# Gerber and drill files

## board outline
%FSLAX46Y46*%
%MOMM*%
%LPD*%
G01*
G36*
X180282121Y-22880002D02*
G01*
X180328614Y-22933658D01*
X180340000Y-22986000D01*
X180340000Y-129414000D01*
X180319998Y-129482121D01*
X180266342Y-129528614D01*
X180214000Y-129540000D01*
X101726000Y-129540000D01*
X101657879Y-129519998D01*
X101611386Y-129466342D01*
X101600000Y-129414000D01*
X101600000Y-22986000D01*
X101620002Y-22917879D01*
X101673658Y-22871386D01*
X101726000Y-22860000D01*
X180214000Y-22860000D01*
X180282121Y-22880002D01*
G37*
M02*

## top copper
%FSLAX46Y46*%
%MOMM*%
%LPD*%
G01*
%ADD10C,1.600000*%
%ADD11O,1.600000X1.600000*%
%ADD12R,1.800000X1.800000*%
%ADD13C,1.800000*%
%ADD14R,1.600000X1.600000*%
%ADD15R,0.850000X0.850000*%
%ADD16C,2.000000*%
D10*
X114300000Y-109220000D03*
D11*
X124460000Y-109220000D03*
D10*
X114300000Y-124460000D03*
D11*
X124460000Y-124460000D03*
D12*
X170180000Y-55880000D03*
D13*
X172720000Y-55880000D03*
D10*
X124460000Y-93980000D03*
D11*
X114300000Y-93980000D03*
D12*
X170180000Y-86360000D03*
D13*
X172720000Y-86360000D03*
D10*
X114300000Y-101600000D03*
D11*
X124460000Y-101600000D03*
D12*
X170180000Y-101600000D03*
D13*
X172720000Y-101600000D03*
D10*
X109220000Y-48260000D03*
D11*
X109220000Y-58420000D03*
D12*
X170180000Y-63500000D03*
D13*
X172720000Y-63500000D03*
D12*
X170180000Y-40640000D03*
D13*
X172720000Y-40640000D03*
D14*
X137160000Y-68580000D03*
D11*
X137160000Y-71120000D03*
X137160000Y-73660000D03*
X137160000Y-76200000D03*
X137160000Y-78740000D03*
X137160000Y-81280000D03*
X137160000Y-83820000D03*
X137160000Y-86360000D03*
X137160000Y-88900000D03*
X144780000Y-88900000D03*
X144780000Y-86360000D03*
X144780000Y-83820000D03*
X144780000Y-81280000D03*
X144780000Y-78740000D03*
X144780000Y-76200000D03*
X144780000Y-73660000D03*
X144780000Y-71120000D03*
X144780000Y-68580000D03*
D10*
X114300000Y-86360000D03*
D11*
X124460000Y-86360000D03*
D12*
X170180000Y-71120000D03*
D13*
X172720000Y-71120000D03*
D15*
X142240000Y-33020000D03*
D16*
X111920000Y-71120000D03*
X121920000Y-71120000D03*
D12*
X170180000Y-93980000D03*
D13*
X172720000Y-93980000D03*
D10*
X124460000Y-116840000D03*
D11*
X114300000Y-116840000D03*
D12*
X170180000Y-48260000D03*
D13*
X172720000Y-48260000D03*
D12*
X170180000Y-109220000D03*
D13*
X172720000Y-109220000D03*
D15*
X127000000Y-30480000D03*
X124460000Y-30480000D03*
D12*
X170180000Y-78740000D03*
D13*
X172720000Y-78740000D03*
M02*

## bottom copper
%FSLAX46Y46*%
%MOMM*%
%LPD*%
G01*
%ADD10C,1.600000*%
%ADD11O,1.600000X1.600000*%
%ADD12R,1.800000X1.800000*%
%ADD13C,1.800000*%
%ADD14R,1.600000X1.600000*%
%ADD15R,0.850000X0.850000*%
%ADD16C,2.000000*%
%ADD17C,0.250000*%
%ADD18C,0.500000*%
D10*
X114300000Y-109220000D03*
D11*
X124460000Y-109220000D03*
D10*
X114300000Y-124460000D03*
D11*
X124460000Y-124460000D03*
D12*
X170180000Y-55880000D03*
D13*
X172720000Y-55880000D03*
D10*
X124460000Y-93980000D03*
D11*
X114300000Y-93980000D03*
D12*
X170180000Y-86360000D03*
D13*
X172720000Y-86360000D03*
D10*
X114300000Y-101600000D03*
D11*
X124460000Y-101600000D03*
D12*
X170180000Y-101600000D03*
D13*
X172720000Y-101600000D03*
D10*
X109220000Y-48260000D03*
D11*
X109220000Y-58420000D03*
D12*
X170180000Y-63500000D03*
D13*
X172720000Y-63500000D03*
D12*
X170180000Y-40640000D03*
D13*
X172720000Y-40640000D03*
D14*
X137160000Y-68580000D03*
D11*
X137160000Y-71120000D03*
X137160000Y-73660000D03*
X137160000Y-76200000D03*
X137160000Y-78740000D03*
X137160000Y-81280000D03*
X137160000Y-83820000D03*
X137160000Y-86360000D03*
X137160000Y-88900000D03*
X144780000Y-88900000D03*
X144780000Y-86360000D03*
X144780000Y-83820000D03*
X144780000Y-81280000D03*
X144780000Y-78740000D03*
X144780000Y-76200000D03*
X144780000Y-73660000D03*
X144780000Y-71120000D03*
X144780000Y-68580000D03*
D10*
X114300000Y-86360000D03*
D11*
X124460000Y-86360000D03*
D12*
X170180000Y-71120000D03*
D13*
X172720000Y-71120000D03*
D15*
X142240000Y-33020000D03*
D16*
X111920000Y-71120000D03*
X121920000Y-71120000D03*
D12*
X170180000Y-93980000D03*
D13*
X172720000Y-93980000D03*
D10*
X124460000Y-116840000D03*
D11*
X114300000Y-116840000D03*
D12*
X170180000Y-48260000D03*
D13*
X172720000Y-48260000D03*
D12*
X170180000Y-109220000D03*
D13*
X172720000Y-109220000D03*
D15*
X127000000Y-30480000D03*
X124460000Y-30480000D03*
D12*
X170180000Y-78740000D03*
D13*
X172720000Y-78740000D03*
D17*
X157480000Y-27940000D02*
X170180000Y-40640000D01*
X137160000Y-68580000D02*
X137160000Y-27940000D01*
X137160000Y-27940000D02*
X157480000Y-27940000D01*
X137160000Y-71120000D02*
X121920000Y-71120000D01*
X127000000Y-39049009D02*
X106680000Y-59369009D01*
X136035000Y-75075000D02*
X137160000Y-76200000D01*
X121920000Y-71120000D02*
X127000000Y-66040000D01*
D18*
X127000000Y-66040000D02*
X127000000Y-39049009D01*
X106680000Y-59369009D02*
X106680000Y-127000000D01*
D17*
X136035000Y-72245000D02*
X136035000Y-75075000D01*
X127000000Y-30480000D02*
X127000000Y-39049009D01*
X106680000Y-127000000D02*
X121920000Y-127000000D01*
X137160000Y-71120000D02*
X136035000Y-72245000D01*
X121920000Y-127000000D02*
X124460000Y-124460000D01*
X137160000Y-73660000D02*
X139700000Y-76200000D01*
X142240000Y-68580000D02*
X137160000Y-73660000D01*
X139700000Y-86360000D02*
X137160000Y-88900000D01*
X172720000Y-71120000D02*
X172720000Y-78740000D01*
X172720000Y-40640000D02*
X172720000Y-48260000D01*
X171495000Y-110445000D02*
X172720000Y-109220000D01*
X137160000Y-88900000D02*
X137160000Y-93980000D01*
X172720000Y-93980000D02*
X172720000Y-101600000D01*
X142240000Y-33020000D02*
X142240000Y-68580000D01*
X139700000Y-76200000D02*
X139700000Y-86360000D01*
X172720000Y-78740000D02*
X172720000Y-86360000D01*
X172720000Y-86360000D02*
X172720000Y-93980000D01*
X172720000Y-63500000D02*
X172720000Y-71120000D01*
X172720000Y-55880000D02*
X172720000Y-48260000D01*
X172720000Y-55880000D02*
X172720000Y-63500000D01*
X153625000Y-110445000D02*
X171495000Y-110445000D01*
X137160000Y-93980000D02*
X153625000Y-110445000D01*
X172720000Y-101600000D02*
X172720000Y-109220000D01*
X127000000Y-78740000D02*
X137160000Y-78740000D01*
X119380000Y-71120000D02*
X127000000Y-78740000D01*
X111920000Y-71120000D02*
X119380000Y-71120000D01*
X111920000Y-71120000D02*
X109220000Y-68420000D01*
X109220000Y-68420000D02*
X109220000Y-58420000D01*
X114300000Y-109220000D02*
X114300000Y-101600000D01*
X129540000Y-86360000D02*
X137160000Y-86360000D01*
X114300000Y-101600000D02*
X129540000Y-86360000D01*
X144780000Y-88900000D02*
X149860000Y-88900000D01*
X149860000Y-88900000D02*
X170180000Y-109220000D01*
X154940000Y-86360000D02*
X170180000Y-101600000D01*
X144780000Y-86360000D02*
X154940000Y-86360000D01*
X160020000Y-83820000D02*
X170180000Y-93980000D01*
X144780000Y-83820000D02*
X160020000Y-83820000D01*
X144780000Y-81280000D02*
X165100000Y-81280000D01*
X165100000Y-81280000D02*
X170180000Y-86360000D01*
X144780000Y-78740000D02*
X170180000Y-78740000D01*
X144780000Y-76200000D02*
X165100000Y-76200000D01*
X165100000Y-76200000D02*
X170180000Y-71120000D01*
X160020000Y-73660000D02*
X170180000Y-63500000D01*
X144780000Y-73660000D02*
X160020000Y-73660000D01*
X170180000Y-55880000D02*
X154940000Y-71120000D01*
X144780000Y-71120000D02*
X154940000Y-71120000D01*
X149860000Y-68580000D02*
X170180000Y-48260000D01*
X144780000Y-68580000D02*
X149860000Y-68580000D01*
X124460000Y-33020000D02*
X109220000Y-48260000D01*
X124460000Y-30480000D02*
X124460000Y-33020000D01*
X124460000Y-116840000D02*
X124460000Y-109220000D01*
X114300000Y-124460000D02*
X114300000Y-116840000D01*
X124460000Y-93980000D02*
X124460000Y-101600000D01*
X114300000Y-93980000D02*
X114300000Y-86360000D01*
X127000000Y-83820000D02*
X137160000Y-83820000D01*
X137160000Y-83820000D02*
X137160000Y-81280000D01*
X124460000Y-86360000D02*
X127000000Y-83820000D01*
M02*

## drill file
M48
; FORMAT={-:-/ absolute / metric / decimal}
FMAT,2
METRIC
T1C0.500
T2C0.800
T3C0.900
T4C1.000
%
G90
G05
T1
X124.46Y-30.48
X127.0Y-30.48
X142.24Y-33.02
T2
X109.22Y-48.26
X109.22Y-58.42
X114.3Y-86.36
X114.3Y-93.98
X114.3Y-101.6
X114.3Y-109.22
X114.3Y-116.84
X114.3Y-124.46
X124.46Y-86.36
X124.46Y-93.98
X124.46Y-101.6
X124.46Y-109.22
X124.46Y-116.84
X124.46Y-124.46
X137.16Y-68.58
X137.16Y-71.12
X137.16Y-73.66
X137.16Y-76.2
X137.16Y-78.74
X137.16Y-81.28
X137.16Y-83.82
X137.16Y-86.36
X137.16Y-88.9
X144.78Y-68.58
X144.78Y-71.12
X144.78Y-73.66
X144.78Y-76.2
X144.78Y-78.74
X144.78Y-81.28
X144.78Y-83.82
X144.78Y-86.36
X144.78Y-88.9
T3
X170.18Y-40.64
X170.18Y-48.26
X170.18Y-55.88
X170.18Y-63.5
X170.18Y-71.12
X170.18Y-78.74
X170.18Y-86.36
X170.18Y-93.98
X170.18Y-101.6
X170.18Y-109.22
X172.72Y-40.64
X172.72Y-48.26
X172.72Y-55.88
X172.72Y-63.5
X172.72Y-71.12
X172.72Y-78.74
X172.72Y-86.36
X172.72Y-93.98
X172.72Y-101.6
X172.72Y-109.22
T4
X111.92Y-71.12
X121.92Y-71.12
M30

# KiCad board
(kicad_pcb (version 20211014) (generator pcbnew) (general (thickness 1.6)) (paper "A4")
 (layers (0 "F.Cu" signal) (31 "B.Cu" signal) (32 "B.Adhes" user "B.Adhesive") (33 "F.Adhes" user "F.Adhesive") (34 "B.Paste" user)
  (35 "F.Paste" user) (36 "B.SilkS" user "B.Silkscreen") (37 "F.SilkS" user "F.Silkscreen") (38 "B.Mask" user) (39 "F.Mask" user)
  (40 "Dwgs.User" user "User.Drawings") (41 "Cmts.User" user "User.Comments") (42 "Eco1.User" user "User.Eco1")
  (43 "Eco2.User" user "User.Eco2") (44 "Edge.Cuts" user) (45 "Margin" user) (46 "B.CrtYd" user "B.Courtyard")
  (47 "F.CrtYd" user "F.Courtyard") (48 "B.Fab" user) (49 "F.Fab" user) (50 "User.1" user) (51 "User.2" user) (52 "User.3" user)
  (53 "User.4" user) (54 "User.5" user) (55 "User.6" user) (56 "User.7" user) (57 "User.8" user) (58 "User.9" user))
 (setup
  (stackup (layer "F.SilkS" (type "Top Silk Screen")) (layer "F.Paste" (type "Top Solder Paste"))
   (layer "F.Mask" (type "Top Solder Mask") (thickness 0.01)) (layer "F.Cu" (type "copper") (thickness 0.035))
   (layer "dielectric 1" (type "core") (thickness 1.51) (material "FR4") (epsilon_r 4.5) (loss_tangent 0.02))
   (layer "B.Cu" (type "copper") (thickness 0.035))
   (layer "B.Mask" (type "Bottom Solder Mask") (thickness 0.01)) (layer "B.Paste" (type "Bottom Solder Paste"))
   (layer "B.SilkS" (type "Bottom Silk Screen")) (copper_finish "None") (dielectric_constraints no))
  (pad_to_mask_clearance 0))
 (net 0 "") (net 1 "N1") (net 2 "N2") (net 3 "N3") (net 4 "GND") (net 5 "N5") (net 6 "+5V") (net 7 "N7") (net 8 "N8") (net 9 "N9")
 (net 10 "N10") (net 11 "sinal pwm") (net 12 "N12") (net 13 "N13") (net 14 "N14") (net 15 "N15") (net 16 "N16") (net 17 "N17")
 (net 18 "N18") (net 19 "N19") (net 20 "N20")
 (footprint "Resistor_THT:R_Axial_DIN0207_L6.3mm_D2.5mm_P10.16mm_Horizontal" (layer "F.Cu") (at 114.3 109.22)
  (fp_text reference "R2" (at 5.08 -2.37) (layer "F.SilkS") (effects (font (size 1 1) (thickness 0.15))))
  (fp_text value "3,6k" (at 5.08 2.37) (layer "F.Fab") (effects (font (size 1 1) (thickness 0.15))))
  (pad "1" thru_hole circle (at 0 0) (size 1.6 1.6) (drill 0.8) (layers *.Cu *.Mask) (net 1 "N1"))
  (pad "2" thru_hole oval (at 10.16 0) (size 1.6 1.6) (drill 0.8) (layers *.Cu *.Mask) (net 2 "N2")))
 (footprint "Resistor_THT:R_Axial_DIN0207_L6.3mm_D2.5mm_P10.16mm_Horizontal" (layer "F.Cu") (at 114.3 124.46)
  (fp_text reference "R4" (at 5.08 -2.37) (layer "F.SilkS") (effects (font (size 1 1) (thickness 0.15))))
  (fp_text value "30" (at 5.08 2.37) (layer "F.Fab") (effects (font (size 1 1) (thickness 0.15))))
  (pad "1" thru_hole circle (at 0 0) (size 1.6 1.6) (drill 0.8) (layers *.Cu *.Mask) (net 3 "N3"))
  (pad "2" thru_hole oval (at 10.16 0) (size 1.6 1.6) (drill 0.8) (layers *.Cu *.Mask) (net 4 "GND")))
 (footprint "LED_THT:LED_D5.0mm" (layer "F.Cu") (at 170.18 55.88)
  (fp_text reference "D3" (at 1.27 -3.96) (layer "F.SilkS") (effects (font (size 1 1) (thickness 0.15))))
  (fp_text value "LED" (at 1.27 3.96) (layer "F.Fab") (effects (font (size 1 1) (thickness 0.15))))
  (pad "1" thru_hole rect (at 0 0) (size 1.8 1.8) (drill 0.9) (layers *.Cu *.Mask) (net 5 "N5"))
  (pad "2" thru_hole circle (at 2.54 0) (size 1.8 1.8) (drill 0.9) (layers *.Cu *.Mask) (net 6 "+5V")))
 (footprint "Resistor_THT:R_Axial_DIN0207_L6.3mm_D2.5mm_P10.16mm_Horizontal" (layer "F.Cu") (at 124.46 93.98 180)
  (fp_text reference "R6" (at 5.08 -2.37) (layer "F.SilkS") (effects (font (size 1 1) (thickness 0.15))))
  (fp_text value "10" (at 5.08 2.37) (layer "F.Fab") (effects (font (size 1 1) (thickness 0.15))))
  (pad "1" thru_hole circle (at 0 0 180) (size 1.6 1.6) (drill 0.8) (layers *.Cu *.Mask) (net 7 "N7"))
  (pad "2" thru_hole oval (at 10.16 0 180) (size 1.6 1.6) (drill 0.8) (layers *.Cu *.Mask) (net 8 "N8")))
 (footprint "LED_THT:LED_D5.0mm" (layer "F.Cu") (at 170.18 86.36)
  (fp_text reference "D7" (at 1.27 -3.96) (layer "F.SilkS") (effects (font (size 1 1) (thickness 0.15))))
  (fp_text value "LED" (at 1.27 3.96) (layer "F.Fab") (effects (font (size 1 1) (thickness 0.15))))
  (pad "1" thru_hole rect (at 0 0) (size 1.8 1.8) (drill 0.9) (layers *.Cu *.Mask) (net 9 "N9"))
  (pad "2" thru_hole circle (at 2.54 0) (size 1.8 1.8) (drill 0.9) (layers *.Cu *.Mask) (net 6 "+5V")))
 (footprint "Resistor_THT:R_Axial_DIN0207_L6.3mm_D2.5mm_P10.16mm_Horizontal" (layer "F.Cu") (at 114.3 101.6)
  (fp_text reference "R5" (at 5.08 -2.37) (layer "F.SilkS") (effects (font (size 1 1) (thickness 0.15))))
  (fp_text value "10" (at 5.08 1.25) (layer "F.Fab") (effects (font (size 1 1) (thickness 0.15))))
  (pad "1" thru_hole circle (at 0 0) (size 1.6 1.6) (drill 0.8) (layers *.Cu *.Mask) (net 1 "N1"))
  (pad "2" thru_hole oval (at 10.16 0) (size 1.6 1.6) (drill 0.8) (layers *.Cu *.Mask) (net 7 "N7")))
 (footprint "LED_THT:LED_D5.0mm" (layer "F.Cu") (at 170.18 101.6)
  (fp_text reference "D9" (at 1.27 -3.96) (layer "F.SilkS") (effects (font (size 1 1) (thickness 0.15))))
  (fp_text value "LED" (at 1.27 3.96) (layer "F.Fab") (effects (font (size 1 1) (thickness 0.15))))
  (pad "1" thru_hole rect (at 0 0) (size 1.8 1.8) (drill 0.9) (layers *.Cu *.Mask) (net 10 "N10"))
  (pad "2" thru_hole circle (at 2.54 0) (size 1.8 1.8) (drill 0.9) (layers *.Cu *.Mask) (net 6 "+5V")))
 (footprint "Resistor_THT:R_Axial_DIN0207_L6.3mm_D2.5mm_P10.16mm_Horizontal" (layer "F.Cu") (at 109.22 48.26 -90)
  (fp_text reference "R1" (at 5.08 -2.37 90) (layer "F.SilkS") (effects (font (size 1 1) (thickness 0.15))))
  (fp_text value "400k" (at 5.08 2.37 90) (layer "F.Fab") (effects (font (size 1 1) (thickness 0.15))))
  (pad "1" thru_hole circle (at 0 0 270) (size 1.6 1.6) (drill 0.8) (layers *.Cu *.Mask) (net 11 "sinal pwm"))
  (pad "2" thru_hole oval (at 10.16 0 270) (size 1.6 1.6) (drill 0.8) (layers *.Cu *.Mask) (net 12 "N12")))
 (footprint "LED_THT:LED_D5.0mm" (layer "F.Cu") (at 170.18 63.5)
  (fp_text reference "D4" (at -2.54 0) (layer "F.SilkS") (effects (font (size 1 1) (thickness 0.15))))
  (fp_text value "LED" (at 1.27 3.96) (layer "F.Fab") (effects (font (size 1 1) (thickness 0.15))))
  (pad "1" thru_hole rect (at 0 0) (size 1.8 1.8) (drill 0.9) (layers *.Cu *.Mask) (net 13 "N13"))
  (pad "2" thru_hole circle (at 2.54 0) (size 1.8 1.8) (drill 0.9) (layers *.Cu *.Mask) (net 6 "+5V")))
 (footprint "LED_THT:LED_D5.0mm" (layer "F.Cu") (at 170.18 40.64)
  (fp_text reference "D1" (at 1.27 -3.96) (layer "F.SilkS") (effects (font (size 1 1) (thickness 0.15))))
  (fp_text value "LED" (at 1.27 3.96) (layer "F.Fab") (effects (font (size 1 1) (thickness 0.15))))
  (pad "1" thru_hole rect (at 0 0) (size 1.8 1.8) (drill 0.9) (layers *.Cu *.Mask) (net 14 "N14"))
  (pad "2" thru_hole circle (at 2.54 0) (size 1.8 1.8) (drill 0.9) (layers *.Cu *.Mask) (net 6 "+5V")))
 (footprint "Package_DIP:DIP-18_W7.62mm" (layer "F.Cu") (at 137.16 68.58)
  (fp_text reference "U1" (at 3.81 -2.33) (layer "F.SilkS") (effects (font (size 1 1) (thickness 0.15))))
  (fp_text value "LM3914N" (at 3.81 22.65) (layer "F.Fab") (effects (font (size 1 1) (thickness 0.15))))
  (pad "1" thru_hole rect (at 0 0) (size 1.6 1.6) (drill 0.8) (layers *.Cu *.Mask) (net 14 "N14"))
  (pad "2" thru_hole oval (at 0 2.54) (size 1.6 1.6) (drill 0.8) (layers *.Cu *.Mask) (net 4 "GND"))
  (pad "3" thru_hole oval (at 0 5.08) (size 1.6 1.6) (drill 0.8) (layers *.Cu *.Mask) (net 6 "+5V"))
  (pad "4" thru_hole oval (at 0 7.62) (size 1.6 1.6) (drill 0.8) (layers *.Cu *.Mask) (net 4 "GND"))
  (pad "5" thru_hole oval (at 0 10.16) (size 1.6 1.6) (drill 0.8) (layers *.Cu *.Mask) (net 12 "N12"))
  (pad "6" thru_hole oval (at 0 12.7) (size 1.6 1.6) (drill 0.8) (layers *.Cu *.Mask) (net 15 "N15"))
  (pad "7" thru_hole oval (at 0 15.24) (size 1.6 1.6) (drill 0.8) (layers *.Cu *.Mask) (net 15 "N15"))
  (pad "8" thru_hole oval (at 0 17.78) (size 1.6 1.6) (drill 0.8) (layers *.Cu *.Mask) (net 1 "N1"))
  (pad "9" thru_hole oval (at 0 20.32) (size 1.6 1.6) (drill 0.8) (layers *.Cu *.Mask) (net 6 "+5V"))
  (pad "10" thru_hole oval (at 7.62 20.32) (size 1.6 1.6) (drill 0.8) (layers *.Cu *.Mask) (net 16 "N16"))
  (pad "11" thru_hole oval (at 7.62 17.78) (size 1.6 1.6) (drill 0.8) (layers *.Cu *.Mask) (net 10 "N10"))
  (pad "12" thru_hole oval (at 7.62 15.24) (size 1.6 1.6) (drill 0.8) (layers *.Cu *.Mask) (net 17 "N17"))
  (pad "13" thru_hole oval (at 7.62 12.7) (size 1.6 1.6) (drill 0.8) (layers *.Cu *.Mask) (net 9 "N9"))
  (pad "14" thru_hole oval (at 7.62 10.16) (size 1.6 1.6) (drill 0.8) (layers *.Cu *.Mask) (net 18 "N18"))
  (pad "15" thru_hole oval (at 7.62 7.62) (size 1.6 1.6) (drill 0.8) (layers *.Cu *.Mask) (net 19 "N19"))
  (pad "16" thru_hole oval (at 7.62 5.08) (size 1.6 1.6) (drill 0.8) (layers *.Cu *.Mask) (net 13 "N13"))
  (pad "17" thru_hole oval (at 7.62 2.54) (size 1.6 1.6) (drill 0.8) (layers *.Cu *.Mask) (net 5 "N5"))
  (pad "18" thru_hole oval (at 7.62 0) (size 1.6 1.6) (drill 0.8) (layers *.Cu *.Mask) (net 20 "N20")))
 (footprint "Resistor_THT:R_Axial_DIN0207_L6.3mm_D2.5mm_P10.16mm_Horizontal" (layer "F.Cu") (at 114.3 86.36)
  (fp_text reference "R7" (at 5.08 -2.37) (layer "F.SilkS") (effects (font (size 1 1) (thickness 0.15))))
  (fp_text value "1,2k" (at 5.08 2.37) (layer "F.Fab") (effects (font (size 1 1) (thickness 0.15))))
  (pad "1" thru_hole circle (at 0 0) (size 1.6 1.6) (drill 0.8) (layers *.Cu *.Mask) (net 8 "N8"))
  (pad "2" thru_hole oval (at 10.16 0) (size 1.6 1.6) (drill 0.8) (layers *.Cu *.Mask) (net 15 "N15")))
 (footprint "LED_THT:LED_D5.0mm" (layer "F.Cu") (at 170.18 71.12)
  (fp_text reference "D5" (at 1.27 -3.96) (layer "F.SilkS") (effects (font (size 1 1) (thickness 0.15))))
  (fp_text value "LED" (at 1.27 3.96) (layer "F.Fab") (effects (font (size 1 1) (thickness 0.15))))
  (pad "1" thru_hole rect (at 0 0) (size 1.8 1.8) (drill 0.9) (layers *.Cu *.Mask) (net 19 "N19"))
  (pad "2" thru_hole circle (at 2.54 0) (size 1.8 1.8) (drill 0.9) (layers *.Cu *.Mask) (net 6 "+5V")))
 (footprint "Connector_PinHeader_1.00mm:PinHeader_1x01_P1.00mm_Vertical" (layer "F.Cu") (at 142.24 33.02)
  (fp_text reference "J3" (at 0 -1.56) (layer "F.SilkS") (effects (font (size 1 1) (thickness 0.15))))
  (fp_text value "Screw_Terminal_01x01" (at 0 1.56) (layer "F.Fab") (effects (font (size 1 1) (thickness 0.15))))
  (pad "1" thru_hole rect (at 0 0) (size 0.85 0.85) (drill 0.5) (layers *.Cu *.Mask) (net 6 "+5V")))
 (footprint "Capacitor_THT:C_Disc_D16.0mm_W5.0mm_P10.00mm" (layer "F.Cu") (at 111.92 71.12)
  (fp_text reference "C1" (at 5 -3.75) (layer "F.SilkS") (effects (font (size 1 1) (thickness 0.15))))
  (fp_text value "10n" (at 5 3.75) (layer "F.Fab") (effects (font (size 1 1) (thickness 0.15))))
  (pad "1" thru_hole circle (at 0 0) (size 2 2) (drill 1) (layers *.Cu *.Mask) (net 12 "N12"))
  (pad "2" thru_hole circle (at 10 0) (size 2 2) (drill 1) (layers *.Cu *.Mask) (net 4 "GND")))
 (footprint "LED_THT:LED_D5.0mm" (layer "F.Cu") (at 170.18 93.98)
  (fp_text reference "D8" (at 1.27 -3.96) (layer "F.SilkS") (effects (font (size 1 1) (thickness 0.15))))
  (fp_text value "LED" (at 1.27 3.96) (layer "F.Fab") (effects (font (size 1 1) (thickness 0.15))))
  (pad "1" thru_hole rect (at 0 0) (size 1.8 1.8) (drill 0.9) (layers *.Cu *.Mask) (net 17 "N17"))
  (pad "2" thru_hole circle (at 2.54 0) (size 1.8 1.8) (drill 0.9) (layers *.Cu *.Mask) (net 6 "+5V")))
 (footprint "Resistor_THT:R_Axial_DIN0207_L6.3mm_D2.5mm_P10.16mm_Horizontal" (layer "F.Cu") (at 124.46 116.84 180)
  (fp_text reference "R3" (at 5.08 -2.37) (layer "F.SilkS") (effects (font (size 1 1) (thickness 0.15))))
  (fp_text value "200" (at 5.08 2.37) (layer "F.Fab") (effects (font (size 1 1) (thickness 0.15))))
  (pad "1" thru_hole circle (at 0 0 180) (size 1.6 1.6) (drill 0.8) (layers *.Cu *.Mask) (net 2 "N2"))
  (pad "2" thru_hole oval (at 10.16 0 180) (size 1.6 1.6) (drill 0.8) (layers *.Cu *.Mask) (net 3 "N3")))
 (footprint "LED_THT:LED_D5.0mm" (layer "F.Cu") (at 170.18 48.26)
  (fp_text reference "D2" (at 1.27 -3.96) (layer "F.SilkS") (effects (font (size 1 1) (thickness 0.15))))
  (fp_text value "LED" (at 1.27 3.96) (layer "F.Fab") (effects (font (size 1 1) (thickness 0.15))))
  (pad "1" thru_hole rect (at 0 0) (size 1.8 1.8) (drill 0.9) (layers *.Cu *.Mask) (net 20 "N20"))
  (pad "2" thru_hole circle (at 2.54 0) (size 1.8 1.8) (drill 0.9) (layers *.Cu *.Mask) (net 6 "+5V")))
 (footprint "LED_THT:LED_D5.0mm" (layer "F.Cu") (at 170.18 109.22)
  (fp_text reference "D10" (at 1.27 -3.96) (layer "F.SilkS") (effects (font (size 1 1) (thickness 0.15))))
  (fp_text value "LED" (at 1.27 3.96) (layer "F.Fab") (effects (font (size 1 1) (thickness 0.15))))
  (pad "1" thru_hole rect (at 0 0) (size 1.8 1.8) (drill 0.9) (layers *.Cu *.Mask) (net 16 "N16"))
  (pad "2" thru_hole circle (at 2.54 0) (size 1.8 1.8) (drill 0.9) (layers *.Cu *.Mask) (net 6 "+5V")))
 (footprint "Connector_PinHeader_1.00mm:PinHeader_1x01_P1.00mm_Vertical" (layer "F.Cu") (at 127 30.48)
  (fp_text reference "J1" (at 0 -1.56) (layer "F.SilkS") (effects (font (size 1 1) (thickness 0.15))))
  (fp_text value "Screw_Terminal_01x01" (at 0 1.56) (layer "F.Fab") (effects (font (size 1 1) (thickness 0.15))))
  (pad "1" thru_hole rect (at 0 0) (size 0.85 0.85) (drill 0.5) (layers *.Cu *.Mask) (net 4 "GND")))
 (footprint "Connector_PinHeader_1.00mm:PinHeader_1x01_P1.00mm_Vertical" (layer "F.Cu") (at 124.46 30.48)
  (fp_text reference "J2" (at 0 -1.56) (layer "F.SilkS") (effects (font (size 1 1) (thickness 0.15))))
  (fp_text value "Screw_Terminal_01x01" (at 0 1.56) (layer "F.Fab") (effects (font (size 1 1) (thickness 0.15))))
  (pad "1" thru_hole rect (at 0 0) (size 0.85 0.85) (drill 0.5) (layers *.Cu *.Mask) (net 11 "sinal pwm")))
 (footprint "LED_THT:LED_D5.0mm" (layer "F.Cu") (at 170.18 78.74)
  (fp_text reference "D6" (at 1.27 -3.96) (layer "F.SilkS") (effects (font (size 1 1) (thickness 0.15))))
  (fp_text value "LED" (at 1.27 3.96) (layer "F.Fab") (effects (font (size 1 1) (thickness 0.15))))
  (pad "1" thru_hole rect (at 0 0) (size 1.8 1.8) (drill 0.9) (layers *.Cu *.Mask) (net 18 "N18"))
  (pad "2" thru_hole circle (at 2.54 0) (size 1.8 1.8) (drill 0.9) (layers *.Cu *.Mask) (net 6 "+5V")))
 (gr_rect (start 177.8 134.62) (end 177.8 134.62) (layer "B.Cu") (width 0.2) (fill none))
 (segment (start 157.48 27.94) (end 170.18 40.64) (width 0.25) (layer "B.Cu") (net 14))
 (segment (start 137.16 68.58) (end 137.16 27.94) (width 0.25) (layer "B.Cu") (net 14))
 (segment (start 137.16 27.94) (end 157.48 27.94) (width 0.25) (layer "B.Cu") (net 14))
 (segment (start 137.16 71.12) (end 121.92 71.12) (width 0.25) (layer "B.Cu") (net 4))
 (segment (start 127 39.049009) (end 106.68 59.369009) (width 0.25) (layer "B.Cu") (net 4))
 (segment (start 136.035 75.075) (end 137.16 76.2) (width 0.25) (layer "B.Cu") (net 4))
 (segment (start 121.92 71.12) (end 127 66.04) (width 0.25) (layer "B.Cu") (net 4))
 (segment (start 127 66.04) (end 127 39.049009) (width 0.5) (layer "B.Cu") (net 4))
 (segment (start 106.68 59.369009) (end 106.68 127) (width 0.5) (layer "B.Cu") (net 4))
 (segment (start 136.035 72.245) (end 136.035 75.075) (width 0.25) (layer "B.Cu") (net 4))
 (segment (start 127 30.48) (end 127 39.049009) (width 0.25) (layer "B.Cu") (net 4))
 (segment (start 106.68 127) (end 121.92 127) (width 0.25) (layer "B.Cu") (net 4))
 (segment (start 137.16 71.12) (end 136.035 72.245) (width 0.25) (layer "B.Cu") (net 4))
 (segment (start 121.92 127) (end 124.46 124.46) (width 0.25) (layer "B.Cu") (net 4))
 (segment (start 137.16 73.66) (end 139.7 76.2) (width 0.25) (layer "B.Cu") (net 6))
 (segment (start 142.24 68.58) (end 137.16 73.66) (width 0.25) (layer "B.Cu") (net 6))
 (segment (start 139.7 86.36) (end 137.16 88.9) (width 0.25) (layer "B.Cu") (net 6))
 (segment (start 172.72 71.12) (end 172.72 78.74) (width 0.25) (layer "B.Cu") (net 6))
 (segment (start 172.72 40.64) (end 172.72 48.26) (width 0.25) (layer "B.Cu") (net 6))
 (segment (start 171.495 110.445) (end 172.72 109.22) (width 0.25) (layer "B.Cu") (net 6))
 (segment (start 137.16 88.9) (end 137.16 93.98) (width 0.25) (layer "B.Cu") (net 6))
 (segment (start 172.72 93.98) (end 172.72 101.6) (width 0.25) (layer "B.Cu") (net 6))
 (segment (start 142.24 33.02) (end 142.24 68.58) (width 0.25) (layer "B.Cu") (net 6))
 (segment (start 139.7 76.2) (end 139.7 86.36) (width 0.25) (layer "B.Cu") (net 6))
 (segment (start 172.72 78.74) (end 172.72 86.36) (width 0.25) (layer "B.Cu") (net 6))
 (segment (start 172.72 86.36) (end 172.72 93.98) (width 0.25) (layer "B.Cu") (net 6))
 (segment (start 172.72 63.5) (end 172.72 71.12) (width 0.25) (layer "B.Cu") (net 6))
 (segment (start 172.72 55.88) (end 172.72 48.26) (width 0.25) (layer "B.Cu") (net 6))
 (segment (start 172.72 55.88) (end 172.72 63.5) (width 0.25) (layer "B.Cu") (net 6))
 (segment (start 153.625 110.445) (end 171.495 110.445) (width 0.25) (layer "B.Cu") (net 6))
 (segment (start 137.16 93.98) (end 153.625 110.445) (width 0.25) (layer "B.Cu") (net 6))
 (segment (start 172.72 101.6) (end 172.72 109.22) (width 0.25) (layer "B.Cu") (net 6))
 (segment (start 127 78.74) (end 137.16 78.74) (width 0.25) (layer "B.Cu") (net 12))
 (segment (start 119.38 71.12) (end 127 78.74) (width 0.25) (layer "B.Cu") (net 12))
 (segment (start 111.92 71.12) (end 119.38 71.12) (width 0.25) (layer "B.Cu") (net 12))
 (segment (start 111.92 71.12) (end 109.22 68.42) (width 0.25) (layer "B.Cu") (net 12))
 (segment (start 109.22 68.42) (end 109.22 58.42) (width 0.25) (layer "B.Cu") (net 12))
 (segment (start 114.3 109.22) (end 114.3 101.6) (width 0.25) (layer "B.Cu") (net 1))
 (segment (start 129.54 86.36) (end 137.16 86.36) (width 0.25) (layer "B.Cu") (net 1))
 (segment (start 114.3 101.6) (end 129.54 86.36) (width 0.25) (layer "B.Cu") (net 1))
 (segment (start 144.78 88.9) (end 149.86 88.9) (width 0.25) (layer "B.Cu") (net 16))
 (segment (start 149.86 88.9) (end 170.18 109.22) (width 0.25) (layer "B.Cu") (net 16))
 (segment (start 154.94 86.36) (end 170.18 101.6) (width 0.25) (layer "B.Cu") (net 10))
 (segment (start 144.78 86.36) (end 154.94 86.36) (width 0.25) (layer "B.Cu") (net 10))
 (segment (start 160.02 83.82) (end 170.18 93.98) (width 0.25) (layer "B.Cu") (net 17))
 (segment (start 144.78 83.82) (end 160.02 83.82) (width 0.25) (layer "B.Cu") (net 17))
 (segment (start 144.78 81.28) (end 165.1 81.28) (width 0.25) (layer "B.Cu") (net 9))
 (segment (start 165.1 81.28) (end 170.18 86.36) (width 0.25) (layer "B.Cu") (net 9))
 (segment (start 144.78 78.74) (end 170.18 78.74) (width 0.25) (layer "B.Cu") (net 18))
 (segment (start 144.78 76.2) (end 165.1 76.2) (width 0.25) (layer "B.Cu") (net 19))
 (segment (start 165.1 76.2) (end 170.18 71.12) (width 0.25) (layer "B.Cu") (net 19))
 (segment (start 160.02 73.66) (end 170.18 63.5) (width 0.25) (layer "B.Cu") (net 13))
 (segment (start 144.78 73.66) (end 160.02 73.66) (width 0.25) (layer "B.Cu") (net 13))
 (segment (start 170.18 55.88) (end 154.94 71.12) (width 0.25) (layer "B.Cu") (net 5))
 (segment (start 144.78 71.12) (end 154.94 71.12) (width 0.25) (layer "B.Cu") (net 5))
 (segment (start 149.86 68.58) (end 170.18 48.26) (width 0.25) (layer "B.Cu") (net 20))
 (segment (start 144.78 68.58) (end 149.86 68.58) (width 0.25) (layer "B.Cu") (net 20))
 (segment (start 124.46 33.02) (end 109.22 48.26) (width 0.25) (layer "B.Cu") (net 11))
 (segment (start 124.46 30.48) (end 124.46 33.02) (width 0.25) (layer "B.Cu") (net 11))
 (segment (start 124.46 116.84) (end 124.46 109.22) (width 0.25) (layer "B.Cu") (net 2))
 (segment (start 114.3 124.46) (end 114.3 116.84) (width 0.25) (layer "B.Cu") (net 3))
 (segment (start 124.46 93.98) (end 124.46 101.6) (width 0.25) (layer "B.Cu") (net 7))
 (segment (start 114.3 93.98) (end 114.3 86.36) (width 0.25) (layer "B.Cu") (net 8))
 (segment (start 127 83.82) (end 137.16 83.82) (width 0.25) (layer "B.Cu") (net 15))
 (segment (start 137.16 83.82) (end 137.16 81.28) (width 0.25) (layer "B.Cu") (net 15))
 (segment (start 124.46 86.36) (end 127 83.82) (width 0.25) (layer "B.Cu") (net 15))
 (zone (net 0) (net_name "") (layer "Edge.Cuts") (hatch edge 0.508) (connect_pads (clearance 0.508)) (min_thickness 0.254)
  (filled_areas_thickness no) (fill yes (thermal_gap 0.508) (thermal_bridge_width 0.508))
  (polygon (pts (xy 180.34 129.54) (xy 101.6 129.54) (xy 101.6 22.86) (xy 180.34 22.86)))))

